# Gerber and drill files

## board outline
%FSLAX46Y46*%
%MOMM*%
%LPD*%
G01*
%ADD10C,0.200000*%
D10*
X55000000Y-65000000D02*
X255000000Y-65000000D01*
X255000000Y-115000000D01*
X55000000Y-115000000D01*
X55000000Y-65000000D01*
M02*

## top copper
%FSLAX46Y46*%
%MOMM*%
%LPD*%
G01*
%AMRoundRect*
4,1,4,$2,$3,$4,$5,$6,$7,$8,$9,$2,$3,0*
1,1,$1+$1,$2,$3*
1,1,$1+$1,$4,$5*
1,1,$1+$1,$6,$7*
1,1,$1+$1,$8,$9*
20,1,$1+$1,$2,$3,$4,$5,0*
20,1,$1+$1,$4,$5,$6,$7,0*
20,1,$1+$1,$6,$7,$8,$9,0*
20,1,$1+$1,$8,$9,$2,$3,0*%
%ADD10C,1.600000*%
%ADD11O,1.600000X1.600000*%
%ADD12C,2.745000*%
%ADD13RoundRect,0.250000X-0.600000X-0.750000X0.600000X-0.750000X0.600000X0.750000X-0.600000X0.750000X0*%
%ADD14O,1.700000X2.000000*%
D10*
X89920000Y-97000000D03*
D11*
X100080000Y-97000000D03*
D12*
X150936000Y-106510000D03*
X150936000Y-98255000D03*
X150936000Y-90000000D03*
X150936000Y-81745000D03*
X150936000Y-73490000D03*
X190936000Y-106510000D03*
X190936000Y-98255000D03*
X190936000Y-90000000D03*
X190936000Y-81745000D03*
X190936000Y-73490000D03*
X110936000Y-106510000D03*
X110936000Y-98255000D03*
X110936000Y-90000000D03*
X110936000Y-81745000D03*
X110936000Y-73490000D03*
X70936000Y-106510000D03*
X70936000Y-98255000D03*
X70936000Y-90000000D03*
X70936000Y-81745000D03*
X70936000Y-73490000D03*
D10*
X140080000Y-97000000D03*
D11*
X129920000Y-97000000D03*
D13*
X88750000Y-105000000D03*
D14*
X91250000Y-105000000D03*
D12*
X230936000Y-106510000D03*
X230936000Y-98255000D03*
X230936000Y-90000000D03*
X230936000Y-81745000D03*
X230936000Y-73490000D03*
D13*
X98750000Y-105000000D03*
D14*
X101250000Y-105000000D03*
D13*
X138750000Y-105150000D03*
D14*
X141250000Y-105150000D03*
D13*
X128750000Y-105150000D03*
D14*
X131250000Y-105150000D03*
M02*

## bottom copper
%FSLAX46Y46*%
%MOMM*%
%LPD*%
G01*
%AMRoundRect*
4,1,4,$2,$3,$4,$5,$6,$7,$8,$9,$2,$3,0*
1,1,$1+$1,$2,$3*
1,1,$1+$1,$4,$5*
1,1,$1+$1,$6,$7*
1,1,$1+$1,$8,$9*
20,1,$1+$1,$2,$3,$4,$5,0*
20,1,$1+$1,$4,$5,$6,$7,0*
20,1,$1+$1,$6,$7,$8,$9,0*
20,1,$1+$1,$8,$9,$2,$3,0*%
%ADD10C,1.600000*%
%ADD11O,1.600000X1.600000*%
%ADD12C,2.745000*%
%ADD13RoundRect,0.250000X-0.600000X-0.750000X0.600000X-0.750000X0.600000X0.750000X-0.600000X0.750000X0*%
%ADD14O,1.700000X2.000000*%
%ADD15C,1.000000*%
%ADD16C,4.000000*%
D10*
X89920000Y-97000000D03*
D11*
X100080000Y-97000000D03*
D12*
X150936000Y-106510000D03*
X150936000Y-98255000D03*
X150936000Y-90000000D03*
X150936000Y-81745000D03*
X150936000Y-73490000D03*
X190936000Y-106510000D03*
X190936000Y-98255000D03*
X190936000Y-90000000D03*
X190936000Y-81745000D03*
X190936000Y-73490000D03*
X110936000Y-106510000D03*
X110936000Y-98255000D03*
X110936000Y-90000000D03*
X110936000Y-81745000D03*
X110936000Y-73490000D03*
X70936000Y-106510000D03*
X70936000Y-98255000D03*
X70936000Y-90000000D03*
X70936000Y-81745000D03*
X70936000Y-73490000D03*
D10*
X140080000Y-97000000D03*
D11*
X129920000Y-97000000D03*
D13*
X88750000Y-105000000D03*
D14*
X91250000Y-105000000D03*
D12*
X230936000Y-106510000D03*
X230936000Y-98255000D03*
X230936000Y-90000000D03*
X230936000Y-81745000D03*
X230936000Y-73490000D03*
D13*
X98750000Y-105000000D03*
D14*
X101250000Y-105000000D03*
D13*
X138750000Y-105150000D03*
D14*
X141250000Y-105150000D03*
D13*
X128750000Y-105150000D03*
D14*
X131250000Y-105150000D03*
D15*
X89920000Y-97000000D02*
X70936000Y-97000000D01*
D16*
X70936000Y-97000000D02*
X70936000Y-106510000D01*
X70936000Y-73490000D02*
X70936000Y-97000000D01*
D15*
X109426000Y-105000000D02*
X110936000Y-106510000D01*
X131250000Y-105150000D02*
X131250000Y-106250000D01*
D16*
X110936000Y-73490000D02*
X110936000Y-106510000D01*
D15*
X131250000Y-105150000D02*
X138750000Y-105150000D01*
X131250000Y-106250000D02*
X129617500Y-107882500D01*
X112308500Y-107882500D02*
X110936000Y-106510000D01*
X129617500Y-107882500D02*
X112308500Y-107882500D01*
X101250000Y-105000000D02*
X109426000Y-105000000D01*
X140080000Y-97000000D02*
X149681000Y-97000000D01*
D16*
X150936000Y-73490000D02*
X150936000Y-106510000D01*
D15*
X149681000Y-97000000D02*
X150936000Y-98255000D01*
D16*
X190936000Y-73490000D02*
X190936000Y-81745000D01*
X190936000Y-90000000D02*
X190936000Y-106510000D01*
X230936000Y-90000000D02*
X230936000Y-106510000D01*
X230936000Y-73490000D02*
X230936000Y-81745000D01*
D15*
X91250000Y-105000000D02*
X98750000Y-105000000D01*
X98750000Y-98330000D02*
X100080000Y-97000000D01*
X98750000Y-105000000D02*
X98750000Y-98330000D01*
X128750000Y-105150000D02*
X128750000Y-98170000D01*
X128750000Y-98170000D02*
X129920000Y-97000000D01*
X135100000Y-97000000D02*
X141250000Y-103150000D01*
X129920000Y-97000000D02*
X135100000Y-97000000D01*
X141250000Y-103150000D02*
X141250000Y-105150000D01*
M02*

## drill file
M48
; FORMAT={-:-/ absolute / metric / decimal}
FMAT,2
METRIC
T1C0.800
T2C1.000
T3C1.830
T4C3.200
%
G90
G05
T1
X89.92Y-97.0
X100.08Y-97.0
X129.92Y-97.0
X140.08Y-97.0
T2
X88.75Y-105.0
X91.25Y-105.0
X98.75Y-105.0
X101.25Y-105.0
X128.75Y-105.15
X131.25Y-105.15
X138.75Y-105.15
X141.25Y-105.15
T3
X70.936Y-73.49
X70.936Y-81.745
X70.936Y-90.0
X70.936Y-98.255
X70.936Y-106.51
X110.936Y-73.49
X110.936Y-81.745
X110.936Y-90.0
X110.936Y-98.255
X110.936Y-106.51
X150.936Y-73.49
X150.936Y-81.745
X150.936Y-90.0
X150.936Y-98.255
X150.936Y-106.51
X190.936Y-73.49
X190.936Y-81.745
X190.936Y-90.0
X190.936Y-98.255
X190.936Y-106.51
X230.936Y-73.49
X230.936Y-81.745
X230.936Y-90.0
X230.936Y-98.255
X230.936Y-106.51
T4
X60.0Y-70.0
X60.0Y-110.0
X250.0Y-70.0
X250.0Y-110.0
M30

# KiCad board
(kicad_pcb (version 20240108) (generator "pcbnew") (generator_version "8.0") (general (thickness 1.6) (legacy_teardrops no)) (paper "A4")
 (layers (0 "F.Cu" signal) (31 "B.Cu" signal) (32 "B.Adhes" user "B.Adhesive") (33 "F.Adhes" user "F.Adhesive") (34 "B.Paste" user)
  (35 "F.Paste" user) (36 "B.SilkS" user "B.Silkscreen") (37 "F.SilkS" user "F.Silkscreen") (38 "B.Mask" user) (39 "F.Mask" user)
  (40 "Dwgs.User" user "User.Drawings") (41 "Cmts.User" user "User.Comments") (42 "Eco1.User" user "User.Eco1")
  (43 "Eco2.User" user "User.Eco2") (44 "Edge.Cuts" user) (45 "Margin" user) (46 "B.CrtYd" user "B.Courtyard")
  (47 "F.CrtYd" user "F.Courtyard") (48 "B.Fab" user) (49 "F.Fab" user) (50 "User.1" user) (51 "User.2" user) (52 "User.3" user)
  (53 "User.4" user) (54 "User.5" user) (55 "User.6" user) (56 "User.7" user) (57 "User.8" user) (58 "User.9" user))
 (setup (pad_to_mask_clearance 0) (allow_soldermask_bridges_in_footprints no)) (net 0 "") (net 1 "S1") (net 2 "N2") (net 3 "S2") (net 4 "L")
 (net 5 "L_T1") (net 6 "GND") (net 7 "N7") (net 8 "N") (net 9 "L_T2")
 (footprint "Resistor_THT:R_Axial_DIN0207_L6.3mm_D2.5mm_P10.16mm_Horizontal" (layer "F.Cu") (at 89.92 97)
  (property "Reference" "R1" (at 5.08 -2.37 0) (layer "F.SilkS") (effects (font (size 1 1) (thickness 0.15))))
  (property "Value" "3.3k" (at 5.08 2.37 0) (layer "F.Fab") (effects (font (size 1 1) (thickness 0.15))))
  (pad "1" thru_hole circle (at 0 0) (size 1.6 1.6) (drill 0.8) (layers "*.Cu" "*.Mask") (remove_unused_layers no) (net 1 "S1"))
  (pad "2" thru_hole oval (at 10.16 0) (size 1.6 1.6) (drill 0.8) (layers "*.Cu" "*.Mask") (remove_unused_layers no) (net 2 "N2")))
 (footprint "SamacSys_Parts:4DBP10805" (layer "F.Cu") (at 150.936 106.51 90)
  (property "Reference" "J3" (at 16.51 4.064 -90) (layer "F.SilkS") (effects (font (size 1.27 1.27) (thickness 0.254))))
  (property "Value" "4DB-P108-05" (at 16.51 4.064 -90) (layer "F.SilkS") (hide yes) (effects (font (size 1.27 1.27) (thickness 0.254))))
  (pad "1" thru_hole circle (at 0 0 90) (size 2.745 2.745) (drill 1.83) (layers "*.Cu" "*.Mask") (remove_unused_layers no) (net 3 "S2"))
  (pad "2" thru_hole circle (at 8.255 0 90) (size 2.745 2.745) (drill 1.83) (layers "*.Cu" "*.Mask") (remove_unused_layers no) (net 3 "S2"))
  (pad "3" thru_hole circle (at 16.51 0 90) (size 2.745 2.745) (drill 1.83) (layers "*.Cu" "*.Mask") (remove_unused_layers no) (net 3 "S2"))
  (pad "4" thru_hole circle (at 24.765 0 90) (size 2.745 2.745) (drill 1.83) (layers "*.Cu" "*.Mask") (remove_unused_layers no) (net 3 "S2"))
  (pad "5" thru_hole circle (at 33.02 0 90) (size 2.745 2.745) (drill 1.83) (layers "*.Cu" "*.Mask") (remove_unused_layers no) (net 3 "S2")))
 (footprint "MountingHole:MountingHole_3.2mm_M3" (layer "F.Cu") (at 60 70)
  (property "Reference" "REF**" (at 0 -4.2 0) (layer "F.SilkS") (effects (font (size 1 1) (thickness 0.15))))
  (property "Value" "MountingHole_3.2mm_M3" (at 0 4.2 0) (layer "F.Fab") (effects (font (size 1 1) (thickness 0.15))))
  (pad "" np_thru_hole circle (at 0 0) (size 3.2 3.2) (drill 3.2) (layers "*.Cu" "*.Mask")))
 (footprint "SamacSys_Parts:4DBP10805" (layer "F.Cu") (at 190.936 106.51 90)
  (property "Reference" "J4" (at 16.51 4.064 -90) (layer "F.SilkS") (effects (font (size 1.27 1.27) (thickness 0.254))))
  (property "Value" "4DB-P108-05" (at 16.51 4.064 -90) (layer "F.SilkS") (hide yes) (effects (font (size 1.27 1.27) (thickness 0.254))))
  (pad "1" thru_hole circle (at 0 0 90) (size 2.745 2.745) (drill 1.83) (layers "*.Cu" "*.Mask") (remove_unused_layers no) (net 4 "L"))
  (pad "2" thru_hole circle (at 8.255 0 90) (size 2.745 2.745) (drill 1.83) (layers "*.Cu" "*.Mask") (remove_unused_layers no) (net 4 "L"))
  (pad "3" thru_hole circle (at 16.51 0 90) (size 2.745 2.745) (drill 1.83) (layers "*.Cu" "*.Mask") (remove_unused_layers no) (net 4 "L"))
  (pad "4" thru_hole circle (at 24.765 0 90) (size 2.745 2.745) (drill 1.83) (layers "*.Cu" "*.Mask") (remove_unused_layers no)
   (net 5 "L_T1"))
  (pad "5" thru_hole circle (at 33.02 0 90) (size 2.745 2.745) (drill 1.83) (layers "*.Cu" "*.Mask") (remove_unused_layers no)
   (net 5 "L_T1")))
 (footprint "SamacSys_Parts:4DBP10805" (layer "F.Cu") (at 110.936 106.51 90)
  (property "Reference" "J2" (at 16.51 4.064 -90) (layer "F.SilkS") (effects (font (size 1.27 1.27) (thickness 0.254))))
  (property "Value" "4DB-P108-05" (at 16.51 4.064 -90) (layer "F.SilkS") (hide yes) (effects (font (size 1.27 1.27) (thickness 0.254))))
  (pad "1" thru_hole circle (at 0 0 90) (size 2.745 2.745) (drill 1.83) (layers "*.Cu" "*.Mask") (remove_unused_layers no) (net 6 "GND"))
  (pad "2" thru_hole circle (at 8.255 0 90) (size 2.745 2.745) (drill 1.83) (layers "*.Cu" "*.Mask") (remove_unused_layers no) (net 6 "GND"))
  (pad "3" thru_hole circle (at 16.51 0 90) (size 2.745 2.745) (drill 1.83) (layers "*.Cu" "*.Mask") (remove_unused_layers no) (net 6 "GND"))
  (pad "4" thru_hole circle (at 24.765 0 90) (size 2.745 2.745) (drill 1.83) (layers "*.Cu" "*.Mask") (remove_unused_layers no)
   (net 6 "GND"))
  (pad "5" thru_hole circle (at 33.02 0 90) (size 2.745 2.745) (drill 1.83) (layers "*.Cu" "*.Mask") (remove_unused_layers no) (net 6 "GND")))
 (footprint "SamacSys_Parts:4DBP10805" (layer "F.Cu") (at 70.936 106.51 90)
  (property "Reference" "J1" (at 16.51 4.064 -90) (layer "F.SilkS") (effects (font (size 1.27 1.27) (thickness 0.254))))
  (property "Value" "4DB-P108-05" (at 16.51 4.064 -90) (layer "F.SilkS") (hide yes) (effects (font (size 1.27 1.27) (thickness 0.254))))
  (pad "1" thru_hole circle (at 0 0 90) (size 2.745 2.745) (drill 1.83) (layers "*.Cu" "*.Mask") (remove_unused_layers no) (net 1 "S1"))
  (pad "2" thru_hole circle (at 8.255 0 90) (size 2.745 2.745) (drill 1.83) (layers "*.Cu" "*.Mask") (remove_unused_layers no) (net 1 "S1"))
  (pad "3" thru_hole circle (at 16.51 0 90) (size 2.745 2.745) (drill 1.83) (layers "*.Cu" "*.Mask") (remove_unused_layers no) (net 1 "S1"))
  (pad "4" thru_hole circle (at 24.765 0 90) (size 2.745 2.745) (drill 1.83) (layers "*.Cu" "*.Mask") (remove_unused_layers no) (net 1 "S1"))
  (pad "5" thru_hole circle (at 33.02 0 90) (size 2.745 2.745) (drill 1.83) (layers "*.Cu" "*.Mask") (remove_unused_layers no) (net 1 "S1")))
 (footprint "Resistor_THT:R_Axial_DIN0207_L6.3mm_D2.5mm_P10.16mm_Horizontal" (layer "F.Cu") (at 140.08 97 180)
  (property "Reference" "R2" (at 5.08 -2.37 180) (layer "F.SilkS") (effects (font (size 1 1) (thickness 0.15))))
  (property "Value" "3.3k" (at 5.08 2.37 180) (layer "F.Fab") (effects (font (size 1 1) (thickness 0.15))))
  (pad "1" thru_hole circle (at 0 0 180) (size 1.6 1.6) (drill 0.8) (layers "*.Cu" "*.Mask") (remove_unused_layers no) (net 3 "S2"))
  (pad "2" thru_hole oval (at 10.16 0 180) (size 1.6 1.6) (drill 0.8) (layers "*.Cu" "*.Mask") (remove_unused_layers no) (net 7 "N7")))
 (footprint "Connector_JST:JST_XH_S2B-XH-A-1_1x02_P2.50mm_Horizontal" (layer "F.Cu") (at 88.75 105)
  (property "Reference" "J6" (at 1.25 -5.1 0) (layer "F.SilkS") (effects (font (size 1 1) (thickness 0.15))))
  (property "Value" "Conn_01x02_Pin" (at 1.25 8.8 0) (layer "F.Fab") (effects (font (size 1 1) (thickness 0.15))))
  (pad "1" thru_hole roundrect (at 0 0) (size 1.7 2) (drill 1) (layers "*.Cu" "*.Mask") (remove_unused_layers no)
   (roundrect_rratio 0.1470588235) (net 6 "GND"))
  (pad "2" thru_hole oval (at 2.5 0) (size 1.7 2) (drill 1) (layers "*.Cu" "*.Mask") (remove_unused_layers no) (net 2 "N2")))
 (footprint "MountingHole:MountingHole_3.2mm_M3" (layer "F.Cu") (at 60 110)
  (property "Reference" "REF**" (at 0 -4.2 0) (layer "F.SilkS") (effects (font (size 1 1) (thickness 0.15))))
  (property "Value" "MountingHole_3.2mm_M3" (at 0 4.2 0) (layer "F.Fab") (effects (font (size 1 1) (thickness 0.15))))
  (pad "" np_thru_hole circle (at 0 0) (size 3.2 3.2) (drill 3.2) (layers "F&B.Cu" "*.Mask")))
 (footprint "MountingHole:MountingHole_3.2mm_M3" (layer "F.Cu") (at 250 110)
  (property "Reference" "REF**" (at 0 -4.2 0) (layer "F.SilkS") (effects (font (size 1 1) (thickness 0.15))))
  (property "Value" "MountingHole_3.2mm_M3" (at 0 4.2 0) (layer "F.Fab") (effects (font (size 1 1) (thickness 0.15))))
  (pad "" np_thru_hole circle (at 0 0) (size 3.2 3.2) (drill 3.2) (layers "F&B.Cu" "*.Mask")))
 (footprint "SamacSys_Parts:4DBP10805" (layer "F.Cu") (at 230.936 106.51 90)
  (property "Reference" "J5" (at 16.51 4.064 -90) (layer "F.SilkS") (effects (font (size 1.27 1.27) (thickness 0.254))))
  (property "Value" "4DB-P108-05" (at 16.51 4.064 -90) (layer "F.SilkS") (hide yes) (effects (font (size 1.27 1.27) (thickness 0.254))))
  (pad "1" thru_hole circle (at 0 0 90) (size 2.745 2.745) (drill 1.83) (layers "*.Cu" "*.Mask") (remove_unused_layers no) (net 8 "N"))
  (pad "2" thru_hole circle (at 8.255 0 90) (size 2.745 2.745) (drill 1.83) (layers "*.Cu" "*.Mask") (remove_unused_layers no) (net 8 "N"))
  (pad "3" thru_hole circle (at 16.51 0 90) (size 2.745 2.745) (drill 1.83) (layers "*.Cu" "*.Mask") (remove_unused_layers no) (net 8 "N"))
  (pad "4" thru_hole circle (at 24.765 0 90) (size 2.745 2.745) (drill 1.83) (layers "*.Cu" "*.Mask") (remove_unused_layers no)
   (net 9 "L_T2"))
  (pad "5" thru_hole circle (at 33.02 0 90) (size 2.745 2.745) (drill 1.83) (layers "*.Cu" "*.Mask") (remove_unused_layers no)
   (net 9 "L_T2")))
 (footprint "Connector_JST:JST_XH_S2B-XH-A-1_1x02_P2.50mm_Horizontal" (layer "F.Cu") (at 98.75 105)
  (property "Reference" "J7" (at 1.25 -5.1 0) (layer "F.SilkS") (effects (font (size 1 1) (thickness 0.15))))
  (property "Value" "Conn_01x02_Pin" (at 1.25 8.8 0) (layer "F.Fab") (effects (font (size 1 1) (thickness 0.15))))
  (pad "1" thru_hole roundrect (at 0 0) (size 1.7 2) (drill 1) (layers "*.Cu" "*.Mask") (remove_unused_layers no)
   (roundrect_rratio 0.1470588235) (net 2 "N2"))
  (pad "2" thru_hole oval (at 2.5 0) (size 1.7 2) (drill 1) (layers "*.Cu" "*.Mask") (remove_unused_layers no) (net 6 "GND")))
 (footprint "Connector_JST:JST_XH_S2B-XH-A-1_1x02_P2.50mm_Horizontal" (layer "F.Cu") (at 138.75 105.15)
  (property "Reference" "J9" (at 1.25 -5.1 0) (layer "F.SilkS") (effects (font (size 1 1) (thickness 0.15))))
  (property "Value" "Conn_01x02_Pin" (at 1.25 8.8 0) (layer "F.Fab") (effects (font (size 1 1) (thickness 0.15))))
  (pad "1" thru_hole roundrect (at 0 0) (size 1.7 2) (drill 1) (layers "*.Cu" "*.Mask") (remove_unused_layers no)
   (roundrect_rratio 0.1470588235) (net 6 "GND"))
  (pad "2" thru_hole oval (at 2.5 0) (size 1.7 2) (drill 1) (layers "*.Cu" "*.Mask") (remove_unused_layers no) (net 7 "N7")))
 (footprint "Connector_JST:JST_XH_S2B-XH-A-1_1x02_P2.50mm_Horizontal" (layer "F.Cu") (at 128.75 105.15)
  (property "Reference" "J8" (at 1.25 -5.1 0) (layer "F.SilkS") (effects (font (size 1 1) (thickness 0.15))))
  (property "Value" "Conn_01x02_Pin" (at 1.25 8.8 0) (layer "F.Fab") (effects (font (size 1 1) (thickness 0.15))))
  (pad "1" thru_hole roundrect (at 0 0) (size 1.7 2) (drill 1) (layers "*.Cu" "*.Mask") (remove_unused_layers no)
   (roundrect_rratio 0.1470588235) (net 7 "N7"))
  (pad "2" thru_hole oval (at 2.5 0) (size 1.7 2) (drill 1) (layers "*.Cu" "*.Mask") (remove_unused_layers no) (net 6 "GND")))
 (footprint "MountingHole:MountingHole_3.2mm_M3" (layer "F.Cu") (at 250 70)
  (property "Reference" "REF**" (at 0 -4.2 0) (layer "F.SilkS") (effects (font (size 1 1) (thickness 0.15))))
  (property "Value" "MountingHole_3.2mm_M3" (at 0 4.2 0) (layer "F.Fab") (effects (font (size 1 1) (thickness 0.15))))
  (pad "" np_thru_hole circle (at 0 0) (size 3.2 3.2) (drill 3.2) (layers "F&B.Cu" "*.Mask")))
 (gr_rect (start 55 65) (end 255 115) (stroke (width 0.2) (type default)) (fill none) (layer "Edge.Cuts"))
 (segment (start 89.92 97) (end 70.936 97) (width 1) (layer "B.Cu") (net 1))
 (segment (start 70.936 97) (end 70.936 106.51) (width 4) (layer "B.Cu") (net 1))
 (segment (start 70.936 73.49) (end 70.936 97) (width 4) (layer "B.Cu") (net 1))
 (segment (start 109.426 105) (end 110.936 106.51) (width 1) (layer "B.Cu") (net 6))
 (segment (start 131.25 105.15) (end 131.25 106.25) (width 1) (layer "B.Cu") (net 6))
 (segment (start 110.936 73.49) (end 110.936 106.51) (width 4) (layer "B.Cu") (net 6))
 (segment (start 131.25 105.15) (end 138.75 105.15) (width 1) (layer "B.Cu") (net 6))
 (segment (start 131.25 106.25) (end 129.6175 107.8825) (width 1) (layer "B.Cu") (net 6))
 (segment (start 112.3085 107.8825) (end 110.936 106.51) (width 1) (layer "B.Cu") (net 6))
 (segment (start 129.6175 107.8825) (end 112.3085 107.8825) (width 1) (layer "B.Cu") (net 6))
 (segment (start 101.25 105) (end 109.426 105) (width 1) (layer "B.Cu") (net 6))
 (segment (start 140.08 97) (end 149.681 97) (width 1) (layer "B.Cu") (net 3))
 (segment (start 150.936 73.49) (end 150.936 106.51) (width 4) (layer "B.Cu") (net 3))
 (segment (start 149.681 97) (end 150.936 98.255) (width 1) (layer "B.Cu") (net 3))
 (segment (start 190.936 73.49) (end 190.936 81.745) (width 4) (layer "B.Cu") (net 5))
 (segment (start 190.936 90) (end 190.936 106.51) (width 4) (layer "B.Cu") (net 4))
 (segment (start 230.936 90) (end 230.936 106.51) (width 4) (layer "B.Cu") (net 8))
 (segment (start 230.936 73.49) (end 230.936 81.745) (width 4) (layer "B.Cu") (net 9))
 (segment (start 91.25 105) (end 98.75 105) (width 1) (layer "B.Cu") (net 2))
 (segment (start 98.75 98.33) (end 100.08 97) (width 1) (layer "B.Cu") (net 2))
 (segment (start 98.75 105) (end 98.75 98.33) (width 1) (layer "B.Cu") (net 2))
 (segment (start 128.75 105.15) (end 128.75 98.17) (width 1) (layer "B.Cu") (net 7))
 (segment (start 128.75 98.17) (end 129.92 97) (width 1) (layer "B.Cu") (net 7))
 (segment (start 135.1 97) (end 141.25 103.15) (width 1) (layer "B.Cu") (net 7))
 (segment (start 129.92 97) (end 135.1 97) (width 1) (layer "B.Cu") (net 7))
 (segment (start 141.25 103.15) (end 141.25 105.15) (width 1) (layer "B.Cu") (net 7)))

